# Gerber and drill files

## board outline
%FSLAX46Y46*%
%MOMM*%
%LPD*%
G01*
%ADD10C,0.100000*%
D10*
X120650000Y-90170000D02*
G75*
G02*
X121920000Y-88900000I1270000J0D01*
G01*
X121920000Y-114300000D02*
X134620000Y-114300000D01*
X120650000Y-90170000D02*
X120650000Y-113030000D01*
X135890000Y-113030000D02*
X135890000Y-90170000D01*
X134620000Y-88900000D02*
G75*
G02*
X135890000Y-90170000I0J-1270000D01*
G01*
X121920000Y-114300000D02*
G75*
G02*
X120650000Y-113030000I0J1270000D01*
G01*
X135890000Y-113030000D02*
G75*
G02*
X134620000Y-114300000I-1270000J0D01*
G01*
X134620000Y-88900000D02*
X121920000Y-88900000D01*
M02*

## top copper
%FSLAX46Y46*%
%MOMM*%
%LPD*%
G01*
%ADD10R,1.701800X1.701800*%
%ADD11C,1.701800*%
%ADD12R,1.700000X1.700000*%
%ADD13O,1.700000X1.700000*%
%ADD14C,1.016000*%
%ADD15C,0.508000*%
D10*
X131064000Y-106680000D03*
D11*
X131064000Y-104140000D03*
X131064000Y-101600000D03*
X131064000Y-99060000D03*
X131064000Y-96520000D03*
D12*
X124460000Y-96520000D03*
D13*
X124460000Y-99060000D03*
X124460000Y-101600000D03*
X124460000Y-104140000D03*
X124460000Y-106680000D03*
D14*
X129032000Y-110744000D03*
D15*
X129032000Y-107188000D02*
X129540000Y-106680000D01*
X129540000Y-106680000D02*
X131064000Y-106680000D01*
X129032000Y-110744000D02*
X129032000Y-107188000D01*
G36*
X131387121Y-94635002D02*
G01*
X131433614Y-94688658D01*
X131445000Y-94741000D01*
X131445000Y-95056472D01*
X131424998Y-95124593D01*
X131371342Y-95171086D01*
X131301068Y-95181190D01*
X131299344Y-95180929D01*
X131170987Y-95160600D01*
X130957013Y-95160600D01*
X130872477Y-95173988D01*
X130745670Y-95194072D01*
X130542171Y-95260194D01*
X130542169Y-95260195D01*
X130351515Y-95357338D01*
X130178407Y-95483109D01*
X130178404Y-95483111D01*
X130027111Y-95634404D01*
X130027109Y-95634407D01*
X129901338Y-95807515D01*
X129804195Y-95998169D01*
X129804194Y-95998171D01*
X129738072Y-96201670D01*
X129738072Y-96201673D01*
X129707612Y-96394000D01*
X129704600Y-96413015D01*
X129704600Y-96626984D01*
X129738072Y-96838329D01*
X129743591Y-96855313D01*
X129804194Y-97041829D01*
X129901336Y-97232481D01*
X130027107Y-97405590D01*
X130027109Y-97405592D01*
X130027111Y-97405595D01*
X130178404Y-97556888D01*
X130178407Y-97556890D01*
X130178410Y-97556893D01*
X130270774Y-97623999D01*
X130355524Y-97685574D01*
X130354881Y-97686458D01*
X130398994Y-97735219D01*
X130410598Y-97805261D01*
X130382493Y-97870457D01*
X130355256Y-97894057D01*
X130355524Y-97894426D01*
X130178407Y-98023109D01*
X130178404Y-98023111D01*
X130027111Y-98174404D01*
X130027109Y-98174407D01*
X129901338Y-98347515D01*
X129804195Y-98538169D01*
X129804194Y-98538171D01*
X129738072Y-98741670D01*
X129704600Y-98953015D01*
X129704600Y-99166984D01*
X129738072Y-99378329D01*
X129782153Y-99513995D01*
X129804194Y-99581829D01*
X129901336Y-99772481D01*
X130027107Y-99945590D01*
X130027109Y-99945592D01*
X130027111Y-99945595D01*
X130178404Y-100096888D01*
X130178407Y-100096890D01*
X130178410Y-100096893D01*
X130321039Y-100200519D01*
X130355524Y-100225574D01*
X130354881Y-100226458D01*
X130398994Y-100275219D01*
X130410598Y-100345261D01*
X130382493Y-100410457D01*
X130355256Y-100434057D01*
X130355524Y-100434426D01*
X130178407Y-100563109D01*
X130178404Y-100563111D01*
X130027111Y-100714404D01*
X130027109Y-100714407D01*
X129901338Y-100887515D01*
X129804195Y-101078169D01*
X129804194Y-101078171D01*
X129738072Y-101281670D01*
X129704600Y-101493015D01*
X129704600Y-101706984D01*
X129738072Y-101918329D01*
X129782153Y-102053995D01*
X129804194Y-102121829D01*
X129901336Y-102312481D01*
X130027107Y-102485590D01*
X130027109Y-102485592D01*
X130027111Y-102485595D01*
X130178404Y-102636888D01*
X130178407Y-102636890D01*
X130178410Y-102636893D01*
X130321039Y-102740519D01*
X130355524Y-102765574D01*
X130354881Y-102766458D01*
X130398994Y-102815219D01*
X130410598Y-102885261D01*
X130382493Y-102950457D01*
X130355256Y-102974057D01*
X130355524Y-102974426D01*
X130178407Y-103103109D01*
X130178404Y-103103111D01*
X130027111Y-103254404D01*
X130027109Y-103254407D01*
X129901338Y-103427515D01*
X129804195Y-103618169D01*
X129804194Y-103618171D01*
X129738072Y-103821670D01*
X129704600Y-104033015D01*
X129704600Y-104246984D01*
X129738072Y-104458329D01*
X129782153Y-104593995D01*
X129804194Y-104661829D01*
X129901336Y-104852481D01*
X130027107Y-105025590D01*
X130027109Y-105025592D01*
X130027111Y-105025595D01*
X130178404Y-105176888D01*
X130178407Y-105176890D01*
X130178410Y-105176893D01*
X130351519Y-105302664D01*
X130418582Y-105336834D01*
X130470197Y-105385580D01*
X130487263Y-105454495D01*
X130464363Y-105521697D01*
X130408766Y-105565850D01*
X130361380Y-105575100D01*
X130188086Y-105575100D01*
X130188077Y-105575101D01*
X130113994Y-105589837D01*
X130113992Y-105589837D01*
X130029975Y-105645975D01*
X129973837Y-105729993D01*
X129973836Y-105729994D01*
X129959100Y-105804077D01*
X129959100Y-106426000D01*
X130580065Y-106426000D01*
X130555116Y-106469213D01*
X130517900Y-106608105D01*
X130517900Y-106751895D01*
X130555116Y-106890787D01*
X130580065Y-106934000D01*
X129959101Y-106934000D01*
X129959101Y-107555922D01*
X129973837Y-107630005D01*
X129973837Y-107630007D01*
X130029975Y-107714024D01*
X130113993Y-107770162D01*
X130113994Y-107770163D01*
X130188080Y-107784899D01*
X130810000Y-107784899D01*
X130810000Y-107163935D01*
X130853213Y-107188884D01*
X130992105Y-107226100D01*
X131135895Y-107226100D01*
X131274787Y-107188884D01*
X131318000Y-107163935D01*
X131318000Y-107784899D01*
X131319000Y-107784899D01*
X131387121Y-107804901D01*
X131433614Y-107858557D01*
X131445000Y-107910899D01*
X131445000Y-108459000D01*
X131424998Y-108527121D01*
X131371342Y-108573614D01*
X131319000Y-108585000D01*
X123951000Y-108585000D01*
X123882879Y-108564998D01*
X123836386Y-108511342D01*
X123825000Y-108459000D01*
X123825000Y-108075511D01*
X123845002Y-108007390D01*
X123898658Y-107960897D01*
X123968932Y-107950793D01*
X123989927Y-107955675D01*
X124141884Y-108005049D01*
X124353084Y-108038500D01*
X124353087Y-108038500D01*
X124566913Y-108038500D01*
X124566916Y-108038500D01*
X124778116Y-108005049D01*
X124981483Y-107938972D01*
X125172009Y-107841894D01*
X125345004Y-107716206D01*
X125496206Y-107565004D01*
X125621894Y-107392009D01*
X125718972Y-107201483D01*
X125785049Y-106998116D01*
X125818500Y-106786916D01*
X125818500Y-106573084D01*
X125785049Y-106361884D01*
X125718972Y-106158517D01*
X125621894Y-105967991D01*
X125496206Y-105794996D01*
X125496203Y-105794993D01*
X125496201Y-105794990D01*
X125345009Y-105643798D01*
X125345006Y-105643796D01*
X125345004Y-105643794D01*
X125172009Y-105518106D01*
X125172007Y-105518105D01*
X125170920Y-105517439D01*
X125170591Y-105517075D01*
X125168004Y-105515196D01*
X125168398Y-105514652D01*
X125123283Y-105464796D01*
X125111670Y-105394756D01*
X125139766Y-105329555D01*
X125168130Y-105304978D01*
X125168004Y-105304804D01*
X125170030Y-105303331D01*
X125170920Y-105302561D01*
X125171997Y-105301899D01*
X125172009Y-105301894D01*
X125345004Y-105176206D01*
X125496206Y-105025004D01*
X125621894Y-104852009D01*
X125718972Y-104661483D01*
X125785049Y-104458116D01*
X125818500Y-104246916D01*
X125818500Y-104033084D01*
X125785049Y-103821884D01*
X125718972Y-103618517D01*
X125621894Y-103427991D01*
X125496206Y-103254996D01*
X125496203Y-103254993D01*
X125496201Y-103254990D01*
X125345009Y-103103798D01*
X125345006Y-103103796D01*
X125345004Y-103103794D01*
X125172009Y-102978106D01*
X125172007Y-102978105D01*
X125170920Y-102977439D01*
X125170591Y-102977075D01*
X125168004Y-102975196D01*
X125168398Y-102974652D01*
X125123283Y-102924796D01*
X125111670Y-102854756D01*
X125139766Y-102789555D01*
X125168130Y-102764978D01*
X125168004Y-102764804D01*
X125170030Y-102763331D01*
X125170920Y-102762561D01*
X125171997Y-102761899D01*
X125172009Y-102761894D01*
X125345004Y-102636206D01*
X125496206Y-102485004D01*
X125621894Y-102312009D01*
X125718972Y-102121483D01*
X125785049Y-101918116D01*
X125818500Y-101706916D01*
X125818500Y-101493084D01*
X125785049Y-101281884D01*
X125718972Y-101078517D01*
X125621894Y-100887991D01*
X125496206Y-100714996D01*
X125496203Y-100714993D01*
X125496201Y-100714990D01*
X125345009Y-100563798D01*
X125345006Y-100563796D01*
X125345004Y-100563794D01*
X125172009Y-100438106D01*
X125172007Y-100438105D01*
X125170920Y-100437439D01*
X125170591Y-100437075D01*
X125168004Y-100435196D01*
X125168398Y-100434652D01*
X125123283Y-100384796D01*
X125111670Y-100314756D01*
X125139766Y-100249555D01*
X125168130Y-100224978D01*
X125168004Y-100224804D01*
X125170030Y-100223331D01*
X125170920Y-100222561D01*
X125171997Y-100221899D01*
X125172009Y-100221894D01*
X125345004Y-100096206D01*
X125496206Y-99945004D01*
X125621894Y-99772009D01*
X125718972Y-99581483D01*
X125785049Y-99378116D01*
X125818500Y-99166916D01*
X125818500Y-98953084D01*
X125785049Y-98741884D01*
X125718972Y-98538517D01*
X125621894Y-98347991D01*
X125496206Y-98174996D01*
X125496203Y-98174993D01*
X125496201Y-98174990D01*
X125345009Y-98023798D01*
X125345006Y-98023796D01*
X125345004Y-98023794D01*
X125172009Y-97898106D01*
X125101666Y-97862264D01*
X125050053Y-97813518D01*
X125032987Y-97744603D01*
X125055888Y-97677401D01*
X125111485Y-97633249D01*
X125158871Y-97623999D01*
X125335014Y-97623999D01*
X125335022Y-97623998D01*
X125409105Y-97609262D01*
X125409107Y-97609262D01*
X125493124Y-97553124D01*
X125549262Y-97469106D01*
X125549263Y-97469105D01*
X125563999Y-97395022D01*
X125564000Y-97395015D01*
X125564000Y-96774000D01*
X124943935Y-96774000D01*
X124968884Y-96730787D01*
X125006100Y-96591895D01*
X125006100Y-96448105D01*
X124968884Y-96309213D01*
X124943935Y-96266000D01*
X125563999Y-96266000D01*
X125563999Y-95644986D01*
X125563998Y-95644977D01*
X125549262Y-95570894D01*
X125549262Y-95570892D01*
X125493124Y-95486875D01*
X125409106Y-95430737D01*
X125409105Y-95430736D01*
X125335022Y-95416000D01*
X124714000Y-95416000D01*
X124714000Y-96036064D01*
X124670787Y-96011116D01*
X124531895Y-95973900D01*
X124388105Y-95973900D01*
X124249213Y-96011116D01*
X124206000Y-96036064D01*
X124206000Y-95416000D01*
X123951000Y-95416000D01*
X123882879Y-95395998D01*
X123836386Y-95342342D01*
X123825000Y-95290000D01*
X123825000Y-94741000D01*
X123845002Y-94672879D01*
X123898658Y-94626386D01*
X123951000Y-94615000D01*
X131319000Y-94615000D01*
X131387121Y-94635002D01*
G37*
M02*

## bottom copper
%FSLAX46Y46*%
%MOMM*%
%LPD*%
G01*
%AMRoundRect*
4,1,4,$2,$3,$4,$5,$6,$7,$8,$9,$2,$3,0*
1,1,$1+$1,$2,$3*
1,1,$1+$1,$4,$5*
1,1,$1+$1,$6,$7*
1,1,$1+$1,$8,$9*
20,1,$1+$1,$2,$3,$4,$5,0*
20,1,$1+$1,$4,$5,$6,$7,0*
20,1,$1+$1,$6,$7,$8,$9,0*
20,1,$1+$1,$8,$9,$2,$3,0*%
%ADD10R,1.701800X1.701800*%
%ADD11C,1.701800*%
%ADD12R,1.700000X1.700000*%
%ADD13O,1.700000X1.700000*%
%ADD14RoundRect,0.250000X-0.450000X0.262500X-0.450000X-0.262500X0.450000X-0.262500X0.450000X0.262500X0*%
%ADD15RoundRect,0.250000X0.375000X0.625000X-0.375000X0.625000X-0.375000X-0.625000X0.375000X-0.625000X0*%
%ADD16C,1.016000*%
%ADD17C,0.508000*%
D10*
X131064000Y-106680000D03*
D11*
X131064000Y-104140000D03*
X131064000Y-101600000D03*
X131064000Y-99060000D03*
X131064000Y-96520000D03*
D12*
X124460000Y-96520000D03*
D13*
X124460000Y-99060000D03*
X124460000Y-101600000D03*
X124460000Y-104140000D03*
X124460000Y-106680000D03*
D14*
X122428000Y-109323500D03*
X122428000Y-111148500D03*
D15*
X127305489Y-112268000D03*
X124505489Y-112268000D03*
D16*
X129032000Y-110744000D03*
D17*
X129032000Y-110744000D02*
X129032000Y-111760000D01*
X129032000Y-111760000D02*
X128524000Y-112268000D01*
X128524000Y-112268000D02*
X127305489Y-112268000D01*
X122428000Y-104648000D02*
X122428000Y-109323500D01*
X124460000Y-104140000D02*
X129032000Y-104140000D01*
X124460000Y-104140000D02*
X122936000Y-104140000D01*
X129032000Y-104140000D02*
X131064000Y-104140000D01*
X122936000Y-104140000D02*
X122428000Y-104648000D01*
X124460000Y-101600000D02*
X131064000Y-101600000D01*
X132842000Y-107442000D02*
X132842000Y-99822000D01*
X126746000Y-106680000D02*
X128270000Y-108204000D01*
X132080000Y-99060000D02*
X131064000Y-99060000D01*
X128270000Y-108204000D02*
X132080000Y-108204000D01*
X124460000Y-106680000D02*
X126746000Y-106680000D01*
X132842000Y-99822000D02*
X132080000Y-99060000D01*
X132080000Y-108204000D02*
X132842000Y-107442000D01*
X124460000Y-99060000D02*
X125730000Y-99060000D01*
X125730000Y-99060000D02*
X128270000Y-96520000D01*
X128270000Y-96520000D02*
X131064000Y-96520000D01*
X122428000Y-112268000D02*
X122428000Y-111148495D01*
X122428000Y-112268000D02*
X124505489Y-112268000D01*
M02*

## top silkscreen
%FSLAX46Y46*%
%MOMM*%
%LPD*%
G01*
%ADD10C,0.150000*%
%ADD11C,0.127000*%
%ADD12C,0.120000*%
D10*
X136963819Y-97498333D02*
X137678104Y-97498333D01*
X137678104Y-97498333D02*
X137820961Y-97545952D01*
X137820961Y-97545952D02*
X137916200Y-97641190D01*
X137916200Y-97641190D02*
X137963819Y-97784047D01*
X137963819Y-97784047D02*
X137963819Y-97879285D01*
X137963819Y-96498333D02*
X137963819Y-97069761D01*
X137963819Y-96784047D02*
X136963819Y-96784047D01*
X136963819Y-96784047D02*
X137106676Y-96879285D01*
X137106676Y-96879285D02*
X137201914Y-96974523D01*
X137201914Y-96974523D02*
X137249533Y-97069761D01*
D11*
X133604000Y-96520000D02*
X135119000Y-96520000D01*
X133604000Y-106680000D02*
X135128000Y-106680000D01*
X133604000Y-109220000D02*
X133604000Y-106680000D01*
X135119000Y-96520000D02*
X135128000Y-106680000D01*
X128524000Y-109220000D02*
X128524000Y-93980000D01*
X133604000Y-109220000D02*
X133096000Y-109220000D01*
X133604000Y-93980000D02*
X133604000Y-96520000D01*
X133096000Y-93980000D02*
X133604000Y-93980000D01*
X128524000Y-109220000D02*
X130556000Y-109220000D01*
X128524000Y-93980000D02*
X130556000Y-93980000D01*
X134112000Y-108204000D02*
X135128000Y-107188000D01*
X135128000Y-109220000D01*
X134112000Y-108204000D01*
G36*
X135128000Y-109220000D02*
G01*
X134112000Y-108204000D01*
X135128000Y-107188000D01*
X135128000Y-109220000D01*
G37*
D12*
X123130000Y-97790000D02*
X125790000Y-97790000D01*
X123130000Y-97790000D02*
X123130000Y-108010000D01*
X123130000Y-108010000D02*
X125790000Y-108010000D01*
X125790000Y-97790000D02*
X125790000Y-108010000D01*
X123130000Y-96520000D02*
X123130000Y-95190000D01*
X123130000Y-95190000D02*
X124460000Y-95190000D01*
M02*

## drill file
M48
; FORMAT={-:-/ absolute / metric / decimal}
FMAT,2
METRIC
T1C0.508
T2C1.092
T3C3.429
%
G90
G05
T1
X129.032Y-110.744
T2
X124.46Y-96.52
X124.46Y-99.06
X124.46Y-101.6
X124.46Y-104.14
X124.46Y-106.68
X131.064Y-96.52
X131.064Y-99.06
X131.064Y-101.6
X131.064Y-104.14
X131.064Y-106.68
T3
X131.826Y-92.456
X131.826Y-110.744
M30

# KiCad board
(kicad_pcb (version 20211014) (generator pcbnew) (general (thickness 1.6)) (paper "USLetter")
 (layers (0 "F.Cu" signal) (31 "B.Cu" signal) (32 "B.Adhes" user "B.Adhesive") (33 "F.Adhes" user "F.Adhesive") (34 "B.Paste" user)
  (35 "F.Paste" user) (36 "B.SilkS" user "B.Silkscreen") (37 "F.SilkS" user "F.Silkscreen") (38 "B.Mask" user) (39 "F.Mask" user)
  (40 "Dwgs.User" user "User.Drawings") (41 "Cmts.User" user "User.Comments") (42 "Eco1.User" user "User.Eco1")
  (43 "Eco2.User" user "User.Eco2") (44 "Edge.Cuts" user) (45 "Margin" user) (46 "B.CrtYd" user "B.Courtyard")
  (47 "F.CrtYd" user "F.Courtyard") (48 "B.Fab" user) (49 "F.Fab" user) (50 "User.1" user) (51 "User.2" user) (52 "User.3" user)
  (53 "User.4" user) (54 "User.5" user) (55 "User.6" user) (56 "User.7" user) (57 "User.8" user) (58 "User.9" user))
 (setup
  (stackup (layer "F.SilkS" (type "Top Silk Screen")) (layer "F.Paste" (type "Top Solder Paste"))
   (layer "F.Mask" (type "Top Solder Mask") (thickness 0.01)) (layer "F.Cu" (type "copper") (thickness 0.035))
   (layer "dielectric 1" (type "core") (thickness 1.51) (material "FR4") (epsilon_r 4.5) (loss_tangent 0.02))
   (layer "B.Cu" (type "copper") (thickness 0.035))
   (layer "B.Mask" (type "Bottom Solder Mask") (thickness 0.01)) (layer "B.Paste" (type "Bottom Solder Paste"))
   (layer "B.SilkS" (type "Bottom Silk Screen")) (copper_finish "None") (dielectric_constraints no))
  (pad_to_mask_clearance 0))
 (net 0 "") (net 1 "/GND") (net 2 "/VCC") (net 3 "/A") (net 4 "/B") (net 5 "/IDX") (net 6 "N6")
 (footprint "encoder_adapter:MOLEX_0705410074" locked (layer "F.Cu") (at 131.064 106.68 -90)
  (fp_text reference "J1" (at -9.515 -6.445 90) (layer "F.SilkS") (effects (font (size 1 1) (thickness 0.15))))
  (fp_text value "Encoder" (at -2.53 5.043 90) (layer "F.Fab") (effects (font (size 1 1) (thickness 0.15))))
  (fp_line (start -10.16 -2.54) (end -10.16 -4.055) (layer "F.SilkS") (width 0.127))
  (fp_line (start 0 -2.54) (end 0 -4.064) (layer "F.SilkS") (width 0.127))
  (fp_line (start 2.54 -2.54) (end 0 -2.54) (layer "F.SilkS") (width 0.127))
  (fp_line (start -10.16 -4.055) (end 0 -4.064) (layer "F.SilkS") (width 0.127))
  (fp_line (start 2.54 2.54) (end -12.7 2.54) (layer "F.SilkS") (width 0.127))
  (fp_line (start 2.54 -2.54) (end 2.54 -2.032) (layer "F.SilkS") (width 0.127))
  (fp_line (start -12.7 -2.54) (end -10.16 -2.54) (layer "F.SilkS") (width 0.127))
  (fp_line (start -12.7 -2.032) (end -12.7 -2.54) (layer "F.SilkS") (width 0.127))
  (fp_line (start 2.54 2.54) (end 2.54 0.508) (layer "F.SilkS") (width 0.127))
  (fp_line (start -12.7 2.54) (end -12.7 0.508) (layer "F.SilkS") (width 0.127))
  (fp_poly (pts (xy 1.524 -3.048) (xy 0.508 -4.064) (xy 2.54 -4.064)) (layer "F.SilkS") (width 0.127) (fill solid))
  (pad "" np_thru_hole circle locked (at 4.064 -0.762 270) (size 1.524 1.524) (drill 3.429) (layers F&B.Cu *.Mask))
  (pad "" np_thru_hole circle locked (at -14.224 -0.762 270) (size 1.524 1.524) (drill 3.429) (layers F&B.Cu *.Mask))
  (pad "1" thru_hole rect locked (at 0 0 270) (size 1.7018 1.7018) (drill 1.0922) (layers *.Cu) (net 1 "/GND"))
  (pad "2" thru_hole circle locked (at -2.54 0 270) (size 1.7018 1.7018) (drill 1.0922) (layers *.Cu) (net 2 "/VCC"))
  (pad "3" thru_hole circle locked (at -5.08 0 270) (size 1.7018 1.7018) (drill 1.0922) (layers *.Cu) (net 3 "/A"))
  (pad "4" thru_hole circle locked (at -7.62 0 270) (size 1.7018 1.7018) (drill 1.0922) (layers *.Cu) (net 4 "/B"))
  (pad "5" thru_hole circle locked (at -10.16 0 270) (size 1.7018 1.7018) (drill 1.0922) (layers *.Cu) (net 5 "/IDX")))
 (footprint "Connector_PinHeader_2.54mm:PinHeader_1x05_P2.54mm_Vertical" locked (layer "F.Cu") (at 124.46 96.52)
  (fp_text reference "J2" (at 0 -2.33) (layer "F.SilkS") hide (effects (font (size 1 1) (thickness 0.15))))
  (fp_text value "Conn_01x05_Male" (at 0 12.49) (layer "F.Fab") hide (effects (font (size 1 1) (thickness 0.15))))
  (fp_line (start -1.33 1.27) (end 1.33 1.27) (layer "F.SilkS") (width 0.12))
  (fp_line (start -1.33 1.27) (end -1.33 11.49) (layer "F.SilkS") (width 0.12))
  (fp_line (start -1.33 11.49) (end 1.33 11.49) (layer "F.SilkS") (width 0.12))
  (fp_line (start 1.33 1.27) (end 1.33 11.49) (layer "F.SilkS") (width 0.12))
  (fp_line (start -1.33 0) (end -1.33 -1.33) (layer "F.SilkS") (width 0.12))
  (fp_line (start -1.33 -1.33) (end 0 -1.33) (layer "F.SilkS") (width 0.12))
  (pad "1" thru_hole rect locked (at 0 0) (size 1.7 1.7) (drill 1.0922) (layers *.Cu *.Mask) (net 1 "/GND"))
  (pad "2" thru_hole oval locked (at 0 2.54) (size 1.7 1.7) (drill 1.0922) (layers *.Cu *.Mask) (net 5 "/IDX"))
  (pad "3" thru_hole oval locked (at 0 5.08) (size 1.7 1.7) (drill 1.0922) (layers *.Cu *.Mask) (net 3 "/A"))
  (pad "4" thru_hole oval locked (at 0 7.62) (size 1.7 1.7) (drill 1.0922) (layers *.Cu *.Mask) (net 2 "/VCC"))
  (pad "5" thru_hole oval locked (at 0 10.16) (size 1.7 1.7) (drill 1.0922) (layers *.Cu *.Mask) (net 4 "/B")))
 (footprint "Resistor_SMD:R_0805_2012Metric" (layer "B.Cu") (at 122.428 110.236 -90)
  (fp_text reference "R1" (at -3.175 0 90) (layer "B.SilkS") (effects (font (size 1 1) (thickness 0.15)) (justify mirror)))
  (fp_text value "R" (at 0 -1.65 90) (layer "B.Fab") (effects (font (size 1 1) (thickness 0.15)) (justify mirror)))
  (pad "1" smd roundrect (at -0.9125 0 270) (size 1.025 1.4) (layers "B.Cu" "B.Paste" "B.Mask") (roundrect_rratio 0.243902) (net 2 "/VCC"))
  (pad "2" smd roundrect (at 0.9125 0 270) (size 1.025 1.4) (layers "B.Cu" "B.Paste" "B.Mask") (roundrect_rratio 0.243902) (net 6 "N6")))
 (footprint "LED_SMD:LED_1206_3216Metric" (layer "B.Cu") (at 125.905489 112.268 180)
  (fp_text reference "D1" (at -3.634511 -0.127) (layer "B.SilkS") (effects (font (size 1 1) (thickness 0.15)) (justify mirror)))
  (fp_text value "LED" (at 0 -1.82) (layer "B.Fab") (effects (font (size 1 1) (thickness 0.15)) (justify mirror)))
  (pad "1" smd roundrect (at -1.4 0 180) (size 1.25 1.75) (layers "B.Cu" "B.Paste" "B.Mask") (roundrect_rratio 0.2) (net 1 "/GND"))
  (pad "2" smd roundrect (at 1.4 0 180) (size 1.25 1.75) (layers "B.Cu" "B.Paste" "B.Mask") (roundrect_rratio 0.2) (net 6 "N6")))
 (gr_arc (start 120.65 90.17) (mid 121.021974 89.271974) (end 121.92 88.9) (layer "Edge.Cuts") (width 0.1))
 (gr_line (start 121.92 114.3) (end 134.62 114.3) (layer "Edge.Cuts") (width 0.1))
 (gr_line (start 120.65 90.17) (end 120.65 113.03) (layer "Edge.Cuts") (width 0.1))
 (gr_line (start 135.89 113.03) (end 135.89 90.17) (layer "Edge.Cuts") (width 0.1))
 (gr_arc (start 134.62 88.9) (mid 135.518026 89.271974) (end 135.89 90.17) (layer "Edge.Cuts") (width 0.1))
 (gr_arc (start 121.92 114.3) (mid 121.021974 113.928026) (end 120.65 113.03) (layer "Edge.Cuts") (width 0.1))
 (gr_arc (start 135.89 113.03) (mid 135.518026 113.928026) (end 134.62 114.3) (layer "Edge.Cuts") (width 0.1))
 (gr_line (start 134.62 88.9) (end 121.92 88.9) (layer "Edge.Cuts") (width 0.1))
 (segment (start 129.032 107.188) (end 129.54 106.68) (width 0.508) (layer "F.Cu") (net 1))
 (segment (start 129.54 106.68) (end 131.064 106.68) (width 0.508) (layer "F.Cu") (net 1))
 (segment (start 129.032 110.744) (end 129.032 107.188) (width 0.508) (layer "F.Cu") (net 1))
 (via (at 129.032 110.744) (size 1.016) (drill 0.508) (layers "F.Cu" "B.Cu") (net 1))
 (segment (start 129.032 110.744) (end 129.032 111.76) (width 0.508) (layer "B.Cu") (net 1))
 (segment (start 129.032 111.76) (end 128.524 112.268) (width 0.508) (layer "B.Cu") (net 1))
 (segment (start 128.524 112.268) (end 127.305489 112.268) (width 0.508) (layer "B.Cu") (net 1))
 (segment (start 122.428 104.648) (end 122.428 109.3235) (width 0.508) (layer "B.Cu") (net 2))
 (segment (start 124.46 104.14) (end 129.032 104.14) (width 0.508) (layer "B.Cu") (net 2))
 (segment (start 124.46 104.14) (end 122.936 104.14) (width 0.508) (layer "B.Cu") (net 2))
 (segment (start 129.032 104.14) (end 131.064 104.14) (width 0.508) (layer "B.Cu") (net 2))
 (segment (start 122.936 104.14) (end 122.428 104.648) (width 0.508) (layer "B.Cu") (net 2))
 (segment (start 124.46 101.6) (end 131.064 101.6) (width 0.508) (layer "B.Cu") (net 3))
 (segment (start 132.842 107.442) (end 132.842 99.822) (width 0.508) (layer "B.Cu") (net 4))
 (segment (start 126.746 106.68) (end 128.27 108.204) (width 0.508) (layer "B.Cu") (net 4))
 (segment (start 132.08 99.06) (end 131.064 99.06) (width 0.508) (layer "B.Cu") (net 4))
 (segment (start 128.27 108.204) (end 132.08 108.204) (width 0.508) (layer "B.Cu") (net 4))
 (segment (start 124.46 106.68) (end 126.746 106.68) (width 0.508) (layer "B.Cu") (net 4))
 (segment (start 132.842 99.822) (end 132.08 99.06) (width 0.508) (layer "B.Cu") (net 4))
 (segment (start 132.08 108.204) (end 132.842 107.442) (width 0.508) (layer "B.Cu") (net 4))
 (segment (start 124.46 99.06) (end 125.73 99.06) (width 0.508) (layer "B.Cu") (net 5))
 (segment (start 125.73 99.06) (end 128.27 96.52) (width 0.508) (layer "B.Cu") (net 5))
 (segment (start 128.27 96.52) (end 131.064 96.52) (width 0.508) (layer "B.Cu") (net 5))
 (segment (start 122.428 112.268) (end 122.428 111.148495) (width 0.508) (layer "B.Cu") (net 6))
 (segment (start 122.428 112.268) (end 124.505489 112.268) (width 0.508) (layer "B.Cu") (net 6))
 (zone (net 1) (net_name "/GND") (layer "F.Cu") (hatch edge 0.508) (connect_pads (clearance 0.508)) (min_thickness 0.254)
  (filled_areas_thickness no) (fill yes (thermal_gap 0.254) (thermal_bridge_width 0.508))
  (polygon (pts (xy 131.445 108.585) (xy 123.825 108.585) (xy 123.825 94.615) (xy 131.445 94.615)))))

